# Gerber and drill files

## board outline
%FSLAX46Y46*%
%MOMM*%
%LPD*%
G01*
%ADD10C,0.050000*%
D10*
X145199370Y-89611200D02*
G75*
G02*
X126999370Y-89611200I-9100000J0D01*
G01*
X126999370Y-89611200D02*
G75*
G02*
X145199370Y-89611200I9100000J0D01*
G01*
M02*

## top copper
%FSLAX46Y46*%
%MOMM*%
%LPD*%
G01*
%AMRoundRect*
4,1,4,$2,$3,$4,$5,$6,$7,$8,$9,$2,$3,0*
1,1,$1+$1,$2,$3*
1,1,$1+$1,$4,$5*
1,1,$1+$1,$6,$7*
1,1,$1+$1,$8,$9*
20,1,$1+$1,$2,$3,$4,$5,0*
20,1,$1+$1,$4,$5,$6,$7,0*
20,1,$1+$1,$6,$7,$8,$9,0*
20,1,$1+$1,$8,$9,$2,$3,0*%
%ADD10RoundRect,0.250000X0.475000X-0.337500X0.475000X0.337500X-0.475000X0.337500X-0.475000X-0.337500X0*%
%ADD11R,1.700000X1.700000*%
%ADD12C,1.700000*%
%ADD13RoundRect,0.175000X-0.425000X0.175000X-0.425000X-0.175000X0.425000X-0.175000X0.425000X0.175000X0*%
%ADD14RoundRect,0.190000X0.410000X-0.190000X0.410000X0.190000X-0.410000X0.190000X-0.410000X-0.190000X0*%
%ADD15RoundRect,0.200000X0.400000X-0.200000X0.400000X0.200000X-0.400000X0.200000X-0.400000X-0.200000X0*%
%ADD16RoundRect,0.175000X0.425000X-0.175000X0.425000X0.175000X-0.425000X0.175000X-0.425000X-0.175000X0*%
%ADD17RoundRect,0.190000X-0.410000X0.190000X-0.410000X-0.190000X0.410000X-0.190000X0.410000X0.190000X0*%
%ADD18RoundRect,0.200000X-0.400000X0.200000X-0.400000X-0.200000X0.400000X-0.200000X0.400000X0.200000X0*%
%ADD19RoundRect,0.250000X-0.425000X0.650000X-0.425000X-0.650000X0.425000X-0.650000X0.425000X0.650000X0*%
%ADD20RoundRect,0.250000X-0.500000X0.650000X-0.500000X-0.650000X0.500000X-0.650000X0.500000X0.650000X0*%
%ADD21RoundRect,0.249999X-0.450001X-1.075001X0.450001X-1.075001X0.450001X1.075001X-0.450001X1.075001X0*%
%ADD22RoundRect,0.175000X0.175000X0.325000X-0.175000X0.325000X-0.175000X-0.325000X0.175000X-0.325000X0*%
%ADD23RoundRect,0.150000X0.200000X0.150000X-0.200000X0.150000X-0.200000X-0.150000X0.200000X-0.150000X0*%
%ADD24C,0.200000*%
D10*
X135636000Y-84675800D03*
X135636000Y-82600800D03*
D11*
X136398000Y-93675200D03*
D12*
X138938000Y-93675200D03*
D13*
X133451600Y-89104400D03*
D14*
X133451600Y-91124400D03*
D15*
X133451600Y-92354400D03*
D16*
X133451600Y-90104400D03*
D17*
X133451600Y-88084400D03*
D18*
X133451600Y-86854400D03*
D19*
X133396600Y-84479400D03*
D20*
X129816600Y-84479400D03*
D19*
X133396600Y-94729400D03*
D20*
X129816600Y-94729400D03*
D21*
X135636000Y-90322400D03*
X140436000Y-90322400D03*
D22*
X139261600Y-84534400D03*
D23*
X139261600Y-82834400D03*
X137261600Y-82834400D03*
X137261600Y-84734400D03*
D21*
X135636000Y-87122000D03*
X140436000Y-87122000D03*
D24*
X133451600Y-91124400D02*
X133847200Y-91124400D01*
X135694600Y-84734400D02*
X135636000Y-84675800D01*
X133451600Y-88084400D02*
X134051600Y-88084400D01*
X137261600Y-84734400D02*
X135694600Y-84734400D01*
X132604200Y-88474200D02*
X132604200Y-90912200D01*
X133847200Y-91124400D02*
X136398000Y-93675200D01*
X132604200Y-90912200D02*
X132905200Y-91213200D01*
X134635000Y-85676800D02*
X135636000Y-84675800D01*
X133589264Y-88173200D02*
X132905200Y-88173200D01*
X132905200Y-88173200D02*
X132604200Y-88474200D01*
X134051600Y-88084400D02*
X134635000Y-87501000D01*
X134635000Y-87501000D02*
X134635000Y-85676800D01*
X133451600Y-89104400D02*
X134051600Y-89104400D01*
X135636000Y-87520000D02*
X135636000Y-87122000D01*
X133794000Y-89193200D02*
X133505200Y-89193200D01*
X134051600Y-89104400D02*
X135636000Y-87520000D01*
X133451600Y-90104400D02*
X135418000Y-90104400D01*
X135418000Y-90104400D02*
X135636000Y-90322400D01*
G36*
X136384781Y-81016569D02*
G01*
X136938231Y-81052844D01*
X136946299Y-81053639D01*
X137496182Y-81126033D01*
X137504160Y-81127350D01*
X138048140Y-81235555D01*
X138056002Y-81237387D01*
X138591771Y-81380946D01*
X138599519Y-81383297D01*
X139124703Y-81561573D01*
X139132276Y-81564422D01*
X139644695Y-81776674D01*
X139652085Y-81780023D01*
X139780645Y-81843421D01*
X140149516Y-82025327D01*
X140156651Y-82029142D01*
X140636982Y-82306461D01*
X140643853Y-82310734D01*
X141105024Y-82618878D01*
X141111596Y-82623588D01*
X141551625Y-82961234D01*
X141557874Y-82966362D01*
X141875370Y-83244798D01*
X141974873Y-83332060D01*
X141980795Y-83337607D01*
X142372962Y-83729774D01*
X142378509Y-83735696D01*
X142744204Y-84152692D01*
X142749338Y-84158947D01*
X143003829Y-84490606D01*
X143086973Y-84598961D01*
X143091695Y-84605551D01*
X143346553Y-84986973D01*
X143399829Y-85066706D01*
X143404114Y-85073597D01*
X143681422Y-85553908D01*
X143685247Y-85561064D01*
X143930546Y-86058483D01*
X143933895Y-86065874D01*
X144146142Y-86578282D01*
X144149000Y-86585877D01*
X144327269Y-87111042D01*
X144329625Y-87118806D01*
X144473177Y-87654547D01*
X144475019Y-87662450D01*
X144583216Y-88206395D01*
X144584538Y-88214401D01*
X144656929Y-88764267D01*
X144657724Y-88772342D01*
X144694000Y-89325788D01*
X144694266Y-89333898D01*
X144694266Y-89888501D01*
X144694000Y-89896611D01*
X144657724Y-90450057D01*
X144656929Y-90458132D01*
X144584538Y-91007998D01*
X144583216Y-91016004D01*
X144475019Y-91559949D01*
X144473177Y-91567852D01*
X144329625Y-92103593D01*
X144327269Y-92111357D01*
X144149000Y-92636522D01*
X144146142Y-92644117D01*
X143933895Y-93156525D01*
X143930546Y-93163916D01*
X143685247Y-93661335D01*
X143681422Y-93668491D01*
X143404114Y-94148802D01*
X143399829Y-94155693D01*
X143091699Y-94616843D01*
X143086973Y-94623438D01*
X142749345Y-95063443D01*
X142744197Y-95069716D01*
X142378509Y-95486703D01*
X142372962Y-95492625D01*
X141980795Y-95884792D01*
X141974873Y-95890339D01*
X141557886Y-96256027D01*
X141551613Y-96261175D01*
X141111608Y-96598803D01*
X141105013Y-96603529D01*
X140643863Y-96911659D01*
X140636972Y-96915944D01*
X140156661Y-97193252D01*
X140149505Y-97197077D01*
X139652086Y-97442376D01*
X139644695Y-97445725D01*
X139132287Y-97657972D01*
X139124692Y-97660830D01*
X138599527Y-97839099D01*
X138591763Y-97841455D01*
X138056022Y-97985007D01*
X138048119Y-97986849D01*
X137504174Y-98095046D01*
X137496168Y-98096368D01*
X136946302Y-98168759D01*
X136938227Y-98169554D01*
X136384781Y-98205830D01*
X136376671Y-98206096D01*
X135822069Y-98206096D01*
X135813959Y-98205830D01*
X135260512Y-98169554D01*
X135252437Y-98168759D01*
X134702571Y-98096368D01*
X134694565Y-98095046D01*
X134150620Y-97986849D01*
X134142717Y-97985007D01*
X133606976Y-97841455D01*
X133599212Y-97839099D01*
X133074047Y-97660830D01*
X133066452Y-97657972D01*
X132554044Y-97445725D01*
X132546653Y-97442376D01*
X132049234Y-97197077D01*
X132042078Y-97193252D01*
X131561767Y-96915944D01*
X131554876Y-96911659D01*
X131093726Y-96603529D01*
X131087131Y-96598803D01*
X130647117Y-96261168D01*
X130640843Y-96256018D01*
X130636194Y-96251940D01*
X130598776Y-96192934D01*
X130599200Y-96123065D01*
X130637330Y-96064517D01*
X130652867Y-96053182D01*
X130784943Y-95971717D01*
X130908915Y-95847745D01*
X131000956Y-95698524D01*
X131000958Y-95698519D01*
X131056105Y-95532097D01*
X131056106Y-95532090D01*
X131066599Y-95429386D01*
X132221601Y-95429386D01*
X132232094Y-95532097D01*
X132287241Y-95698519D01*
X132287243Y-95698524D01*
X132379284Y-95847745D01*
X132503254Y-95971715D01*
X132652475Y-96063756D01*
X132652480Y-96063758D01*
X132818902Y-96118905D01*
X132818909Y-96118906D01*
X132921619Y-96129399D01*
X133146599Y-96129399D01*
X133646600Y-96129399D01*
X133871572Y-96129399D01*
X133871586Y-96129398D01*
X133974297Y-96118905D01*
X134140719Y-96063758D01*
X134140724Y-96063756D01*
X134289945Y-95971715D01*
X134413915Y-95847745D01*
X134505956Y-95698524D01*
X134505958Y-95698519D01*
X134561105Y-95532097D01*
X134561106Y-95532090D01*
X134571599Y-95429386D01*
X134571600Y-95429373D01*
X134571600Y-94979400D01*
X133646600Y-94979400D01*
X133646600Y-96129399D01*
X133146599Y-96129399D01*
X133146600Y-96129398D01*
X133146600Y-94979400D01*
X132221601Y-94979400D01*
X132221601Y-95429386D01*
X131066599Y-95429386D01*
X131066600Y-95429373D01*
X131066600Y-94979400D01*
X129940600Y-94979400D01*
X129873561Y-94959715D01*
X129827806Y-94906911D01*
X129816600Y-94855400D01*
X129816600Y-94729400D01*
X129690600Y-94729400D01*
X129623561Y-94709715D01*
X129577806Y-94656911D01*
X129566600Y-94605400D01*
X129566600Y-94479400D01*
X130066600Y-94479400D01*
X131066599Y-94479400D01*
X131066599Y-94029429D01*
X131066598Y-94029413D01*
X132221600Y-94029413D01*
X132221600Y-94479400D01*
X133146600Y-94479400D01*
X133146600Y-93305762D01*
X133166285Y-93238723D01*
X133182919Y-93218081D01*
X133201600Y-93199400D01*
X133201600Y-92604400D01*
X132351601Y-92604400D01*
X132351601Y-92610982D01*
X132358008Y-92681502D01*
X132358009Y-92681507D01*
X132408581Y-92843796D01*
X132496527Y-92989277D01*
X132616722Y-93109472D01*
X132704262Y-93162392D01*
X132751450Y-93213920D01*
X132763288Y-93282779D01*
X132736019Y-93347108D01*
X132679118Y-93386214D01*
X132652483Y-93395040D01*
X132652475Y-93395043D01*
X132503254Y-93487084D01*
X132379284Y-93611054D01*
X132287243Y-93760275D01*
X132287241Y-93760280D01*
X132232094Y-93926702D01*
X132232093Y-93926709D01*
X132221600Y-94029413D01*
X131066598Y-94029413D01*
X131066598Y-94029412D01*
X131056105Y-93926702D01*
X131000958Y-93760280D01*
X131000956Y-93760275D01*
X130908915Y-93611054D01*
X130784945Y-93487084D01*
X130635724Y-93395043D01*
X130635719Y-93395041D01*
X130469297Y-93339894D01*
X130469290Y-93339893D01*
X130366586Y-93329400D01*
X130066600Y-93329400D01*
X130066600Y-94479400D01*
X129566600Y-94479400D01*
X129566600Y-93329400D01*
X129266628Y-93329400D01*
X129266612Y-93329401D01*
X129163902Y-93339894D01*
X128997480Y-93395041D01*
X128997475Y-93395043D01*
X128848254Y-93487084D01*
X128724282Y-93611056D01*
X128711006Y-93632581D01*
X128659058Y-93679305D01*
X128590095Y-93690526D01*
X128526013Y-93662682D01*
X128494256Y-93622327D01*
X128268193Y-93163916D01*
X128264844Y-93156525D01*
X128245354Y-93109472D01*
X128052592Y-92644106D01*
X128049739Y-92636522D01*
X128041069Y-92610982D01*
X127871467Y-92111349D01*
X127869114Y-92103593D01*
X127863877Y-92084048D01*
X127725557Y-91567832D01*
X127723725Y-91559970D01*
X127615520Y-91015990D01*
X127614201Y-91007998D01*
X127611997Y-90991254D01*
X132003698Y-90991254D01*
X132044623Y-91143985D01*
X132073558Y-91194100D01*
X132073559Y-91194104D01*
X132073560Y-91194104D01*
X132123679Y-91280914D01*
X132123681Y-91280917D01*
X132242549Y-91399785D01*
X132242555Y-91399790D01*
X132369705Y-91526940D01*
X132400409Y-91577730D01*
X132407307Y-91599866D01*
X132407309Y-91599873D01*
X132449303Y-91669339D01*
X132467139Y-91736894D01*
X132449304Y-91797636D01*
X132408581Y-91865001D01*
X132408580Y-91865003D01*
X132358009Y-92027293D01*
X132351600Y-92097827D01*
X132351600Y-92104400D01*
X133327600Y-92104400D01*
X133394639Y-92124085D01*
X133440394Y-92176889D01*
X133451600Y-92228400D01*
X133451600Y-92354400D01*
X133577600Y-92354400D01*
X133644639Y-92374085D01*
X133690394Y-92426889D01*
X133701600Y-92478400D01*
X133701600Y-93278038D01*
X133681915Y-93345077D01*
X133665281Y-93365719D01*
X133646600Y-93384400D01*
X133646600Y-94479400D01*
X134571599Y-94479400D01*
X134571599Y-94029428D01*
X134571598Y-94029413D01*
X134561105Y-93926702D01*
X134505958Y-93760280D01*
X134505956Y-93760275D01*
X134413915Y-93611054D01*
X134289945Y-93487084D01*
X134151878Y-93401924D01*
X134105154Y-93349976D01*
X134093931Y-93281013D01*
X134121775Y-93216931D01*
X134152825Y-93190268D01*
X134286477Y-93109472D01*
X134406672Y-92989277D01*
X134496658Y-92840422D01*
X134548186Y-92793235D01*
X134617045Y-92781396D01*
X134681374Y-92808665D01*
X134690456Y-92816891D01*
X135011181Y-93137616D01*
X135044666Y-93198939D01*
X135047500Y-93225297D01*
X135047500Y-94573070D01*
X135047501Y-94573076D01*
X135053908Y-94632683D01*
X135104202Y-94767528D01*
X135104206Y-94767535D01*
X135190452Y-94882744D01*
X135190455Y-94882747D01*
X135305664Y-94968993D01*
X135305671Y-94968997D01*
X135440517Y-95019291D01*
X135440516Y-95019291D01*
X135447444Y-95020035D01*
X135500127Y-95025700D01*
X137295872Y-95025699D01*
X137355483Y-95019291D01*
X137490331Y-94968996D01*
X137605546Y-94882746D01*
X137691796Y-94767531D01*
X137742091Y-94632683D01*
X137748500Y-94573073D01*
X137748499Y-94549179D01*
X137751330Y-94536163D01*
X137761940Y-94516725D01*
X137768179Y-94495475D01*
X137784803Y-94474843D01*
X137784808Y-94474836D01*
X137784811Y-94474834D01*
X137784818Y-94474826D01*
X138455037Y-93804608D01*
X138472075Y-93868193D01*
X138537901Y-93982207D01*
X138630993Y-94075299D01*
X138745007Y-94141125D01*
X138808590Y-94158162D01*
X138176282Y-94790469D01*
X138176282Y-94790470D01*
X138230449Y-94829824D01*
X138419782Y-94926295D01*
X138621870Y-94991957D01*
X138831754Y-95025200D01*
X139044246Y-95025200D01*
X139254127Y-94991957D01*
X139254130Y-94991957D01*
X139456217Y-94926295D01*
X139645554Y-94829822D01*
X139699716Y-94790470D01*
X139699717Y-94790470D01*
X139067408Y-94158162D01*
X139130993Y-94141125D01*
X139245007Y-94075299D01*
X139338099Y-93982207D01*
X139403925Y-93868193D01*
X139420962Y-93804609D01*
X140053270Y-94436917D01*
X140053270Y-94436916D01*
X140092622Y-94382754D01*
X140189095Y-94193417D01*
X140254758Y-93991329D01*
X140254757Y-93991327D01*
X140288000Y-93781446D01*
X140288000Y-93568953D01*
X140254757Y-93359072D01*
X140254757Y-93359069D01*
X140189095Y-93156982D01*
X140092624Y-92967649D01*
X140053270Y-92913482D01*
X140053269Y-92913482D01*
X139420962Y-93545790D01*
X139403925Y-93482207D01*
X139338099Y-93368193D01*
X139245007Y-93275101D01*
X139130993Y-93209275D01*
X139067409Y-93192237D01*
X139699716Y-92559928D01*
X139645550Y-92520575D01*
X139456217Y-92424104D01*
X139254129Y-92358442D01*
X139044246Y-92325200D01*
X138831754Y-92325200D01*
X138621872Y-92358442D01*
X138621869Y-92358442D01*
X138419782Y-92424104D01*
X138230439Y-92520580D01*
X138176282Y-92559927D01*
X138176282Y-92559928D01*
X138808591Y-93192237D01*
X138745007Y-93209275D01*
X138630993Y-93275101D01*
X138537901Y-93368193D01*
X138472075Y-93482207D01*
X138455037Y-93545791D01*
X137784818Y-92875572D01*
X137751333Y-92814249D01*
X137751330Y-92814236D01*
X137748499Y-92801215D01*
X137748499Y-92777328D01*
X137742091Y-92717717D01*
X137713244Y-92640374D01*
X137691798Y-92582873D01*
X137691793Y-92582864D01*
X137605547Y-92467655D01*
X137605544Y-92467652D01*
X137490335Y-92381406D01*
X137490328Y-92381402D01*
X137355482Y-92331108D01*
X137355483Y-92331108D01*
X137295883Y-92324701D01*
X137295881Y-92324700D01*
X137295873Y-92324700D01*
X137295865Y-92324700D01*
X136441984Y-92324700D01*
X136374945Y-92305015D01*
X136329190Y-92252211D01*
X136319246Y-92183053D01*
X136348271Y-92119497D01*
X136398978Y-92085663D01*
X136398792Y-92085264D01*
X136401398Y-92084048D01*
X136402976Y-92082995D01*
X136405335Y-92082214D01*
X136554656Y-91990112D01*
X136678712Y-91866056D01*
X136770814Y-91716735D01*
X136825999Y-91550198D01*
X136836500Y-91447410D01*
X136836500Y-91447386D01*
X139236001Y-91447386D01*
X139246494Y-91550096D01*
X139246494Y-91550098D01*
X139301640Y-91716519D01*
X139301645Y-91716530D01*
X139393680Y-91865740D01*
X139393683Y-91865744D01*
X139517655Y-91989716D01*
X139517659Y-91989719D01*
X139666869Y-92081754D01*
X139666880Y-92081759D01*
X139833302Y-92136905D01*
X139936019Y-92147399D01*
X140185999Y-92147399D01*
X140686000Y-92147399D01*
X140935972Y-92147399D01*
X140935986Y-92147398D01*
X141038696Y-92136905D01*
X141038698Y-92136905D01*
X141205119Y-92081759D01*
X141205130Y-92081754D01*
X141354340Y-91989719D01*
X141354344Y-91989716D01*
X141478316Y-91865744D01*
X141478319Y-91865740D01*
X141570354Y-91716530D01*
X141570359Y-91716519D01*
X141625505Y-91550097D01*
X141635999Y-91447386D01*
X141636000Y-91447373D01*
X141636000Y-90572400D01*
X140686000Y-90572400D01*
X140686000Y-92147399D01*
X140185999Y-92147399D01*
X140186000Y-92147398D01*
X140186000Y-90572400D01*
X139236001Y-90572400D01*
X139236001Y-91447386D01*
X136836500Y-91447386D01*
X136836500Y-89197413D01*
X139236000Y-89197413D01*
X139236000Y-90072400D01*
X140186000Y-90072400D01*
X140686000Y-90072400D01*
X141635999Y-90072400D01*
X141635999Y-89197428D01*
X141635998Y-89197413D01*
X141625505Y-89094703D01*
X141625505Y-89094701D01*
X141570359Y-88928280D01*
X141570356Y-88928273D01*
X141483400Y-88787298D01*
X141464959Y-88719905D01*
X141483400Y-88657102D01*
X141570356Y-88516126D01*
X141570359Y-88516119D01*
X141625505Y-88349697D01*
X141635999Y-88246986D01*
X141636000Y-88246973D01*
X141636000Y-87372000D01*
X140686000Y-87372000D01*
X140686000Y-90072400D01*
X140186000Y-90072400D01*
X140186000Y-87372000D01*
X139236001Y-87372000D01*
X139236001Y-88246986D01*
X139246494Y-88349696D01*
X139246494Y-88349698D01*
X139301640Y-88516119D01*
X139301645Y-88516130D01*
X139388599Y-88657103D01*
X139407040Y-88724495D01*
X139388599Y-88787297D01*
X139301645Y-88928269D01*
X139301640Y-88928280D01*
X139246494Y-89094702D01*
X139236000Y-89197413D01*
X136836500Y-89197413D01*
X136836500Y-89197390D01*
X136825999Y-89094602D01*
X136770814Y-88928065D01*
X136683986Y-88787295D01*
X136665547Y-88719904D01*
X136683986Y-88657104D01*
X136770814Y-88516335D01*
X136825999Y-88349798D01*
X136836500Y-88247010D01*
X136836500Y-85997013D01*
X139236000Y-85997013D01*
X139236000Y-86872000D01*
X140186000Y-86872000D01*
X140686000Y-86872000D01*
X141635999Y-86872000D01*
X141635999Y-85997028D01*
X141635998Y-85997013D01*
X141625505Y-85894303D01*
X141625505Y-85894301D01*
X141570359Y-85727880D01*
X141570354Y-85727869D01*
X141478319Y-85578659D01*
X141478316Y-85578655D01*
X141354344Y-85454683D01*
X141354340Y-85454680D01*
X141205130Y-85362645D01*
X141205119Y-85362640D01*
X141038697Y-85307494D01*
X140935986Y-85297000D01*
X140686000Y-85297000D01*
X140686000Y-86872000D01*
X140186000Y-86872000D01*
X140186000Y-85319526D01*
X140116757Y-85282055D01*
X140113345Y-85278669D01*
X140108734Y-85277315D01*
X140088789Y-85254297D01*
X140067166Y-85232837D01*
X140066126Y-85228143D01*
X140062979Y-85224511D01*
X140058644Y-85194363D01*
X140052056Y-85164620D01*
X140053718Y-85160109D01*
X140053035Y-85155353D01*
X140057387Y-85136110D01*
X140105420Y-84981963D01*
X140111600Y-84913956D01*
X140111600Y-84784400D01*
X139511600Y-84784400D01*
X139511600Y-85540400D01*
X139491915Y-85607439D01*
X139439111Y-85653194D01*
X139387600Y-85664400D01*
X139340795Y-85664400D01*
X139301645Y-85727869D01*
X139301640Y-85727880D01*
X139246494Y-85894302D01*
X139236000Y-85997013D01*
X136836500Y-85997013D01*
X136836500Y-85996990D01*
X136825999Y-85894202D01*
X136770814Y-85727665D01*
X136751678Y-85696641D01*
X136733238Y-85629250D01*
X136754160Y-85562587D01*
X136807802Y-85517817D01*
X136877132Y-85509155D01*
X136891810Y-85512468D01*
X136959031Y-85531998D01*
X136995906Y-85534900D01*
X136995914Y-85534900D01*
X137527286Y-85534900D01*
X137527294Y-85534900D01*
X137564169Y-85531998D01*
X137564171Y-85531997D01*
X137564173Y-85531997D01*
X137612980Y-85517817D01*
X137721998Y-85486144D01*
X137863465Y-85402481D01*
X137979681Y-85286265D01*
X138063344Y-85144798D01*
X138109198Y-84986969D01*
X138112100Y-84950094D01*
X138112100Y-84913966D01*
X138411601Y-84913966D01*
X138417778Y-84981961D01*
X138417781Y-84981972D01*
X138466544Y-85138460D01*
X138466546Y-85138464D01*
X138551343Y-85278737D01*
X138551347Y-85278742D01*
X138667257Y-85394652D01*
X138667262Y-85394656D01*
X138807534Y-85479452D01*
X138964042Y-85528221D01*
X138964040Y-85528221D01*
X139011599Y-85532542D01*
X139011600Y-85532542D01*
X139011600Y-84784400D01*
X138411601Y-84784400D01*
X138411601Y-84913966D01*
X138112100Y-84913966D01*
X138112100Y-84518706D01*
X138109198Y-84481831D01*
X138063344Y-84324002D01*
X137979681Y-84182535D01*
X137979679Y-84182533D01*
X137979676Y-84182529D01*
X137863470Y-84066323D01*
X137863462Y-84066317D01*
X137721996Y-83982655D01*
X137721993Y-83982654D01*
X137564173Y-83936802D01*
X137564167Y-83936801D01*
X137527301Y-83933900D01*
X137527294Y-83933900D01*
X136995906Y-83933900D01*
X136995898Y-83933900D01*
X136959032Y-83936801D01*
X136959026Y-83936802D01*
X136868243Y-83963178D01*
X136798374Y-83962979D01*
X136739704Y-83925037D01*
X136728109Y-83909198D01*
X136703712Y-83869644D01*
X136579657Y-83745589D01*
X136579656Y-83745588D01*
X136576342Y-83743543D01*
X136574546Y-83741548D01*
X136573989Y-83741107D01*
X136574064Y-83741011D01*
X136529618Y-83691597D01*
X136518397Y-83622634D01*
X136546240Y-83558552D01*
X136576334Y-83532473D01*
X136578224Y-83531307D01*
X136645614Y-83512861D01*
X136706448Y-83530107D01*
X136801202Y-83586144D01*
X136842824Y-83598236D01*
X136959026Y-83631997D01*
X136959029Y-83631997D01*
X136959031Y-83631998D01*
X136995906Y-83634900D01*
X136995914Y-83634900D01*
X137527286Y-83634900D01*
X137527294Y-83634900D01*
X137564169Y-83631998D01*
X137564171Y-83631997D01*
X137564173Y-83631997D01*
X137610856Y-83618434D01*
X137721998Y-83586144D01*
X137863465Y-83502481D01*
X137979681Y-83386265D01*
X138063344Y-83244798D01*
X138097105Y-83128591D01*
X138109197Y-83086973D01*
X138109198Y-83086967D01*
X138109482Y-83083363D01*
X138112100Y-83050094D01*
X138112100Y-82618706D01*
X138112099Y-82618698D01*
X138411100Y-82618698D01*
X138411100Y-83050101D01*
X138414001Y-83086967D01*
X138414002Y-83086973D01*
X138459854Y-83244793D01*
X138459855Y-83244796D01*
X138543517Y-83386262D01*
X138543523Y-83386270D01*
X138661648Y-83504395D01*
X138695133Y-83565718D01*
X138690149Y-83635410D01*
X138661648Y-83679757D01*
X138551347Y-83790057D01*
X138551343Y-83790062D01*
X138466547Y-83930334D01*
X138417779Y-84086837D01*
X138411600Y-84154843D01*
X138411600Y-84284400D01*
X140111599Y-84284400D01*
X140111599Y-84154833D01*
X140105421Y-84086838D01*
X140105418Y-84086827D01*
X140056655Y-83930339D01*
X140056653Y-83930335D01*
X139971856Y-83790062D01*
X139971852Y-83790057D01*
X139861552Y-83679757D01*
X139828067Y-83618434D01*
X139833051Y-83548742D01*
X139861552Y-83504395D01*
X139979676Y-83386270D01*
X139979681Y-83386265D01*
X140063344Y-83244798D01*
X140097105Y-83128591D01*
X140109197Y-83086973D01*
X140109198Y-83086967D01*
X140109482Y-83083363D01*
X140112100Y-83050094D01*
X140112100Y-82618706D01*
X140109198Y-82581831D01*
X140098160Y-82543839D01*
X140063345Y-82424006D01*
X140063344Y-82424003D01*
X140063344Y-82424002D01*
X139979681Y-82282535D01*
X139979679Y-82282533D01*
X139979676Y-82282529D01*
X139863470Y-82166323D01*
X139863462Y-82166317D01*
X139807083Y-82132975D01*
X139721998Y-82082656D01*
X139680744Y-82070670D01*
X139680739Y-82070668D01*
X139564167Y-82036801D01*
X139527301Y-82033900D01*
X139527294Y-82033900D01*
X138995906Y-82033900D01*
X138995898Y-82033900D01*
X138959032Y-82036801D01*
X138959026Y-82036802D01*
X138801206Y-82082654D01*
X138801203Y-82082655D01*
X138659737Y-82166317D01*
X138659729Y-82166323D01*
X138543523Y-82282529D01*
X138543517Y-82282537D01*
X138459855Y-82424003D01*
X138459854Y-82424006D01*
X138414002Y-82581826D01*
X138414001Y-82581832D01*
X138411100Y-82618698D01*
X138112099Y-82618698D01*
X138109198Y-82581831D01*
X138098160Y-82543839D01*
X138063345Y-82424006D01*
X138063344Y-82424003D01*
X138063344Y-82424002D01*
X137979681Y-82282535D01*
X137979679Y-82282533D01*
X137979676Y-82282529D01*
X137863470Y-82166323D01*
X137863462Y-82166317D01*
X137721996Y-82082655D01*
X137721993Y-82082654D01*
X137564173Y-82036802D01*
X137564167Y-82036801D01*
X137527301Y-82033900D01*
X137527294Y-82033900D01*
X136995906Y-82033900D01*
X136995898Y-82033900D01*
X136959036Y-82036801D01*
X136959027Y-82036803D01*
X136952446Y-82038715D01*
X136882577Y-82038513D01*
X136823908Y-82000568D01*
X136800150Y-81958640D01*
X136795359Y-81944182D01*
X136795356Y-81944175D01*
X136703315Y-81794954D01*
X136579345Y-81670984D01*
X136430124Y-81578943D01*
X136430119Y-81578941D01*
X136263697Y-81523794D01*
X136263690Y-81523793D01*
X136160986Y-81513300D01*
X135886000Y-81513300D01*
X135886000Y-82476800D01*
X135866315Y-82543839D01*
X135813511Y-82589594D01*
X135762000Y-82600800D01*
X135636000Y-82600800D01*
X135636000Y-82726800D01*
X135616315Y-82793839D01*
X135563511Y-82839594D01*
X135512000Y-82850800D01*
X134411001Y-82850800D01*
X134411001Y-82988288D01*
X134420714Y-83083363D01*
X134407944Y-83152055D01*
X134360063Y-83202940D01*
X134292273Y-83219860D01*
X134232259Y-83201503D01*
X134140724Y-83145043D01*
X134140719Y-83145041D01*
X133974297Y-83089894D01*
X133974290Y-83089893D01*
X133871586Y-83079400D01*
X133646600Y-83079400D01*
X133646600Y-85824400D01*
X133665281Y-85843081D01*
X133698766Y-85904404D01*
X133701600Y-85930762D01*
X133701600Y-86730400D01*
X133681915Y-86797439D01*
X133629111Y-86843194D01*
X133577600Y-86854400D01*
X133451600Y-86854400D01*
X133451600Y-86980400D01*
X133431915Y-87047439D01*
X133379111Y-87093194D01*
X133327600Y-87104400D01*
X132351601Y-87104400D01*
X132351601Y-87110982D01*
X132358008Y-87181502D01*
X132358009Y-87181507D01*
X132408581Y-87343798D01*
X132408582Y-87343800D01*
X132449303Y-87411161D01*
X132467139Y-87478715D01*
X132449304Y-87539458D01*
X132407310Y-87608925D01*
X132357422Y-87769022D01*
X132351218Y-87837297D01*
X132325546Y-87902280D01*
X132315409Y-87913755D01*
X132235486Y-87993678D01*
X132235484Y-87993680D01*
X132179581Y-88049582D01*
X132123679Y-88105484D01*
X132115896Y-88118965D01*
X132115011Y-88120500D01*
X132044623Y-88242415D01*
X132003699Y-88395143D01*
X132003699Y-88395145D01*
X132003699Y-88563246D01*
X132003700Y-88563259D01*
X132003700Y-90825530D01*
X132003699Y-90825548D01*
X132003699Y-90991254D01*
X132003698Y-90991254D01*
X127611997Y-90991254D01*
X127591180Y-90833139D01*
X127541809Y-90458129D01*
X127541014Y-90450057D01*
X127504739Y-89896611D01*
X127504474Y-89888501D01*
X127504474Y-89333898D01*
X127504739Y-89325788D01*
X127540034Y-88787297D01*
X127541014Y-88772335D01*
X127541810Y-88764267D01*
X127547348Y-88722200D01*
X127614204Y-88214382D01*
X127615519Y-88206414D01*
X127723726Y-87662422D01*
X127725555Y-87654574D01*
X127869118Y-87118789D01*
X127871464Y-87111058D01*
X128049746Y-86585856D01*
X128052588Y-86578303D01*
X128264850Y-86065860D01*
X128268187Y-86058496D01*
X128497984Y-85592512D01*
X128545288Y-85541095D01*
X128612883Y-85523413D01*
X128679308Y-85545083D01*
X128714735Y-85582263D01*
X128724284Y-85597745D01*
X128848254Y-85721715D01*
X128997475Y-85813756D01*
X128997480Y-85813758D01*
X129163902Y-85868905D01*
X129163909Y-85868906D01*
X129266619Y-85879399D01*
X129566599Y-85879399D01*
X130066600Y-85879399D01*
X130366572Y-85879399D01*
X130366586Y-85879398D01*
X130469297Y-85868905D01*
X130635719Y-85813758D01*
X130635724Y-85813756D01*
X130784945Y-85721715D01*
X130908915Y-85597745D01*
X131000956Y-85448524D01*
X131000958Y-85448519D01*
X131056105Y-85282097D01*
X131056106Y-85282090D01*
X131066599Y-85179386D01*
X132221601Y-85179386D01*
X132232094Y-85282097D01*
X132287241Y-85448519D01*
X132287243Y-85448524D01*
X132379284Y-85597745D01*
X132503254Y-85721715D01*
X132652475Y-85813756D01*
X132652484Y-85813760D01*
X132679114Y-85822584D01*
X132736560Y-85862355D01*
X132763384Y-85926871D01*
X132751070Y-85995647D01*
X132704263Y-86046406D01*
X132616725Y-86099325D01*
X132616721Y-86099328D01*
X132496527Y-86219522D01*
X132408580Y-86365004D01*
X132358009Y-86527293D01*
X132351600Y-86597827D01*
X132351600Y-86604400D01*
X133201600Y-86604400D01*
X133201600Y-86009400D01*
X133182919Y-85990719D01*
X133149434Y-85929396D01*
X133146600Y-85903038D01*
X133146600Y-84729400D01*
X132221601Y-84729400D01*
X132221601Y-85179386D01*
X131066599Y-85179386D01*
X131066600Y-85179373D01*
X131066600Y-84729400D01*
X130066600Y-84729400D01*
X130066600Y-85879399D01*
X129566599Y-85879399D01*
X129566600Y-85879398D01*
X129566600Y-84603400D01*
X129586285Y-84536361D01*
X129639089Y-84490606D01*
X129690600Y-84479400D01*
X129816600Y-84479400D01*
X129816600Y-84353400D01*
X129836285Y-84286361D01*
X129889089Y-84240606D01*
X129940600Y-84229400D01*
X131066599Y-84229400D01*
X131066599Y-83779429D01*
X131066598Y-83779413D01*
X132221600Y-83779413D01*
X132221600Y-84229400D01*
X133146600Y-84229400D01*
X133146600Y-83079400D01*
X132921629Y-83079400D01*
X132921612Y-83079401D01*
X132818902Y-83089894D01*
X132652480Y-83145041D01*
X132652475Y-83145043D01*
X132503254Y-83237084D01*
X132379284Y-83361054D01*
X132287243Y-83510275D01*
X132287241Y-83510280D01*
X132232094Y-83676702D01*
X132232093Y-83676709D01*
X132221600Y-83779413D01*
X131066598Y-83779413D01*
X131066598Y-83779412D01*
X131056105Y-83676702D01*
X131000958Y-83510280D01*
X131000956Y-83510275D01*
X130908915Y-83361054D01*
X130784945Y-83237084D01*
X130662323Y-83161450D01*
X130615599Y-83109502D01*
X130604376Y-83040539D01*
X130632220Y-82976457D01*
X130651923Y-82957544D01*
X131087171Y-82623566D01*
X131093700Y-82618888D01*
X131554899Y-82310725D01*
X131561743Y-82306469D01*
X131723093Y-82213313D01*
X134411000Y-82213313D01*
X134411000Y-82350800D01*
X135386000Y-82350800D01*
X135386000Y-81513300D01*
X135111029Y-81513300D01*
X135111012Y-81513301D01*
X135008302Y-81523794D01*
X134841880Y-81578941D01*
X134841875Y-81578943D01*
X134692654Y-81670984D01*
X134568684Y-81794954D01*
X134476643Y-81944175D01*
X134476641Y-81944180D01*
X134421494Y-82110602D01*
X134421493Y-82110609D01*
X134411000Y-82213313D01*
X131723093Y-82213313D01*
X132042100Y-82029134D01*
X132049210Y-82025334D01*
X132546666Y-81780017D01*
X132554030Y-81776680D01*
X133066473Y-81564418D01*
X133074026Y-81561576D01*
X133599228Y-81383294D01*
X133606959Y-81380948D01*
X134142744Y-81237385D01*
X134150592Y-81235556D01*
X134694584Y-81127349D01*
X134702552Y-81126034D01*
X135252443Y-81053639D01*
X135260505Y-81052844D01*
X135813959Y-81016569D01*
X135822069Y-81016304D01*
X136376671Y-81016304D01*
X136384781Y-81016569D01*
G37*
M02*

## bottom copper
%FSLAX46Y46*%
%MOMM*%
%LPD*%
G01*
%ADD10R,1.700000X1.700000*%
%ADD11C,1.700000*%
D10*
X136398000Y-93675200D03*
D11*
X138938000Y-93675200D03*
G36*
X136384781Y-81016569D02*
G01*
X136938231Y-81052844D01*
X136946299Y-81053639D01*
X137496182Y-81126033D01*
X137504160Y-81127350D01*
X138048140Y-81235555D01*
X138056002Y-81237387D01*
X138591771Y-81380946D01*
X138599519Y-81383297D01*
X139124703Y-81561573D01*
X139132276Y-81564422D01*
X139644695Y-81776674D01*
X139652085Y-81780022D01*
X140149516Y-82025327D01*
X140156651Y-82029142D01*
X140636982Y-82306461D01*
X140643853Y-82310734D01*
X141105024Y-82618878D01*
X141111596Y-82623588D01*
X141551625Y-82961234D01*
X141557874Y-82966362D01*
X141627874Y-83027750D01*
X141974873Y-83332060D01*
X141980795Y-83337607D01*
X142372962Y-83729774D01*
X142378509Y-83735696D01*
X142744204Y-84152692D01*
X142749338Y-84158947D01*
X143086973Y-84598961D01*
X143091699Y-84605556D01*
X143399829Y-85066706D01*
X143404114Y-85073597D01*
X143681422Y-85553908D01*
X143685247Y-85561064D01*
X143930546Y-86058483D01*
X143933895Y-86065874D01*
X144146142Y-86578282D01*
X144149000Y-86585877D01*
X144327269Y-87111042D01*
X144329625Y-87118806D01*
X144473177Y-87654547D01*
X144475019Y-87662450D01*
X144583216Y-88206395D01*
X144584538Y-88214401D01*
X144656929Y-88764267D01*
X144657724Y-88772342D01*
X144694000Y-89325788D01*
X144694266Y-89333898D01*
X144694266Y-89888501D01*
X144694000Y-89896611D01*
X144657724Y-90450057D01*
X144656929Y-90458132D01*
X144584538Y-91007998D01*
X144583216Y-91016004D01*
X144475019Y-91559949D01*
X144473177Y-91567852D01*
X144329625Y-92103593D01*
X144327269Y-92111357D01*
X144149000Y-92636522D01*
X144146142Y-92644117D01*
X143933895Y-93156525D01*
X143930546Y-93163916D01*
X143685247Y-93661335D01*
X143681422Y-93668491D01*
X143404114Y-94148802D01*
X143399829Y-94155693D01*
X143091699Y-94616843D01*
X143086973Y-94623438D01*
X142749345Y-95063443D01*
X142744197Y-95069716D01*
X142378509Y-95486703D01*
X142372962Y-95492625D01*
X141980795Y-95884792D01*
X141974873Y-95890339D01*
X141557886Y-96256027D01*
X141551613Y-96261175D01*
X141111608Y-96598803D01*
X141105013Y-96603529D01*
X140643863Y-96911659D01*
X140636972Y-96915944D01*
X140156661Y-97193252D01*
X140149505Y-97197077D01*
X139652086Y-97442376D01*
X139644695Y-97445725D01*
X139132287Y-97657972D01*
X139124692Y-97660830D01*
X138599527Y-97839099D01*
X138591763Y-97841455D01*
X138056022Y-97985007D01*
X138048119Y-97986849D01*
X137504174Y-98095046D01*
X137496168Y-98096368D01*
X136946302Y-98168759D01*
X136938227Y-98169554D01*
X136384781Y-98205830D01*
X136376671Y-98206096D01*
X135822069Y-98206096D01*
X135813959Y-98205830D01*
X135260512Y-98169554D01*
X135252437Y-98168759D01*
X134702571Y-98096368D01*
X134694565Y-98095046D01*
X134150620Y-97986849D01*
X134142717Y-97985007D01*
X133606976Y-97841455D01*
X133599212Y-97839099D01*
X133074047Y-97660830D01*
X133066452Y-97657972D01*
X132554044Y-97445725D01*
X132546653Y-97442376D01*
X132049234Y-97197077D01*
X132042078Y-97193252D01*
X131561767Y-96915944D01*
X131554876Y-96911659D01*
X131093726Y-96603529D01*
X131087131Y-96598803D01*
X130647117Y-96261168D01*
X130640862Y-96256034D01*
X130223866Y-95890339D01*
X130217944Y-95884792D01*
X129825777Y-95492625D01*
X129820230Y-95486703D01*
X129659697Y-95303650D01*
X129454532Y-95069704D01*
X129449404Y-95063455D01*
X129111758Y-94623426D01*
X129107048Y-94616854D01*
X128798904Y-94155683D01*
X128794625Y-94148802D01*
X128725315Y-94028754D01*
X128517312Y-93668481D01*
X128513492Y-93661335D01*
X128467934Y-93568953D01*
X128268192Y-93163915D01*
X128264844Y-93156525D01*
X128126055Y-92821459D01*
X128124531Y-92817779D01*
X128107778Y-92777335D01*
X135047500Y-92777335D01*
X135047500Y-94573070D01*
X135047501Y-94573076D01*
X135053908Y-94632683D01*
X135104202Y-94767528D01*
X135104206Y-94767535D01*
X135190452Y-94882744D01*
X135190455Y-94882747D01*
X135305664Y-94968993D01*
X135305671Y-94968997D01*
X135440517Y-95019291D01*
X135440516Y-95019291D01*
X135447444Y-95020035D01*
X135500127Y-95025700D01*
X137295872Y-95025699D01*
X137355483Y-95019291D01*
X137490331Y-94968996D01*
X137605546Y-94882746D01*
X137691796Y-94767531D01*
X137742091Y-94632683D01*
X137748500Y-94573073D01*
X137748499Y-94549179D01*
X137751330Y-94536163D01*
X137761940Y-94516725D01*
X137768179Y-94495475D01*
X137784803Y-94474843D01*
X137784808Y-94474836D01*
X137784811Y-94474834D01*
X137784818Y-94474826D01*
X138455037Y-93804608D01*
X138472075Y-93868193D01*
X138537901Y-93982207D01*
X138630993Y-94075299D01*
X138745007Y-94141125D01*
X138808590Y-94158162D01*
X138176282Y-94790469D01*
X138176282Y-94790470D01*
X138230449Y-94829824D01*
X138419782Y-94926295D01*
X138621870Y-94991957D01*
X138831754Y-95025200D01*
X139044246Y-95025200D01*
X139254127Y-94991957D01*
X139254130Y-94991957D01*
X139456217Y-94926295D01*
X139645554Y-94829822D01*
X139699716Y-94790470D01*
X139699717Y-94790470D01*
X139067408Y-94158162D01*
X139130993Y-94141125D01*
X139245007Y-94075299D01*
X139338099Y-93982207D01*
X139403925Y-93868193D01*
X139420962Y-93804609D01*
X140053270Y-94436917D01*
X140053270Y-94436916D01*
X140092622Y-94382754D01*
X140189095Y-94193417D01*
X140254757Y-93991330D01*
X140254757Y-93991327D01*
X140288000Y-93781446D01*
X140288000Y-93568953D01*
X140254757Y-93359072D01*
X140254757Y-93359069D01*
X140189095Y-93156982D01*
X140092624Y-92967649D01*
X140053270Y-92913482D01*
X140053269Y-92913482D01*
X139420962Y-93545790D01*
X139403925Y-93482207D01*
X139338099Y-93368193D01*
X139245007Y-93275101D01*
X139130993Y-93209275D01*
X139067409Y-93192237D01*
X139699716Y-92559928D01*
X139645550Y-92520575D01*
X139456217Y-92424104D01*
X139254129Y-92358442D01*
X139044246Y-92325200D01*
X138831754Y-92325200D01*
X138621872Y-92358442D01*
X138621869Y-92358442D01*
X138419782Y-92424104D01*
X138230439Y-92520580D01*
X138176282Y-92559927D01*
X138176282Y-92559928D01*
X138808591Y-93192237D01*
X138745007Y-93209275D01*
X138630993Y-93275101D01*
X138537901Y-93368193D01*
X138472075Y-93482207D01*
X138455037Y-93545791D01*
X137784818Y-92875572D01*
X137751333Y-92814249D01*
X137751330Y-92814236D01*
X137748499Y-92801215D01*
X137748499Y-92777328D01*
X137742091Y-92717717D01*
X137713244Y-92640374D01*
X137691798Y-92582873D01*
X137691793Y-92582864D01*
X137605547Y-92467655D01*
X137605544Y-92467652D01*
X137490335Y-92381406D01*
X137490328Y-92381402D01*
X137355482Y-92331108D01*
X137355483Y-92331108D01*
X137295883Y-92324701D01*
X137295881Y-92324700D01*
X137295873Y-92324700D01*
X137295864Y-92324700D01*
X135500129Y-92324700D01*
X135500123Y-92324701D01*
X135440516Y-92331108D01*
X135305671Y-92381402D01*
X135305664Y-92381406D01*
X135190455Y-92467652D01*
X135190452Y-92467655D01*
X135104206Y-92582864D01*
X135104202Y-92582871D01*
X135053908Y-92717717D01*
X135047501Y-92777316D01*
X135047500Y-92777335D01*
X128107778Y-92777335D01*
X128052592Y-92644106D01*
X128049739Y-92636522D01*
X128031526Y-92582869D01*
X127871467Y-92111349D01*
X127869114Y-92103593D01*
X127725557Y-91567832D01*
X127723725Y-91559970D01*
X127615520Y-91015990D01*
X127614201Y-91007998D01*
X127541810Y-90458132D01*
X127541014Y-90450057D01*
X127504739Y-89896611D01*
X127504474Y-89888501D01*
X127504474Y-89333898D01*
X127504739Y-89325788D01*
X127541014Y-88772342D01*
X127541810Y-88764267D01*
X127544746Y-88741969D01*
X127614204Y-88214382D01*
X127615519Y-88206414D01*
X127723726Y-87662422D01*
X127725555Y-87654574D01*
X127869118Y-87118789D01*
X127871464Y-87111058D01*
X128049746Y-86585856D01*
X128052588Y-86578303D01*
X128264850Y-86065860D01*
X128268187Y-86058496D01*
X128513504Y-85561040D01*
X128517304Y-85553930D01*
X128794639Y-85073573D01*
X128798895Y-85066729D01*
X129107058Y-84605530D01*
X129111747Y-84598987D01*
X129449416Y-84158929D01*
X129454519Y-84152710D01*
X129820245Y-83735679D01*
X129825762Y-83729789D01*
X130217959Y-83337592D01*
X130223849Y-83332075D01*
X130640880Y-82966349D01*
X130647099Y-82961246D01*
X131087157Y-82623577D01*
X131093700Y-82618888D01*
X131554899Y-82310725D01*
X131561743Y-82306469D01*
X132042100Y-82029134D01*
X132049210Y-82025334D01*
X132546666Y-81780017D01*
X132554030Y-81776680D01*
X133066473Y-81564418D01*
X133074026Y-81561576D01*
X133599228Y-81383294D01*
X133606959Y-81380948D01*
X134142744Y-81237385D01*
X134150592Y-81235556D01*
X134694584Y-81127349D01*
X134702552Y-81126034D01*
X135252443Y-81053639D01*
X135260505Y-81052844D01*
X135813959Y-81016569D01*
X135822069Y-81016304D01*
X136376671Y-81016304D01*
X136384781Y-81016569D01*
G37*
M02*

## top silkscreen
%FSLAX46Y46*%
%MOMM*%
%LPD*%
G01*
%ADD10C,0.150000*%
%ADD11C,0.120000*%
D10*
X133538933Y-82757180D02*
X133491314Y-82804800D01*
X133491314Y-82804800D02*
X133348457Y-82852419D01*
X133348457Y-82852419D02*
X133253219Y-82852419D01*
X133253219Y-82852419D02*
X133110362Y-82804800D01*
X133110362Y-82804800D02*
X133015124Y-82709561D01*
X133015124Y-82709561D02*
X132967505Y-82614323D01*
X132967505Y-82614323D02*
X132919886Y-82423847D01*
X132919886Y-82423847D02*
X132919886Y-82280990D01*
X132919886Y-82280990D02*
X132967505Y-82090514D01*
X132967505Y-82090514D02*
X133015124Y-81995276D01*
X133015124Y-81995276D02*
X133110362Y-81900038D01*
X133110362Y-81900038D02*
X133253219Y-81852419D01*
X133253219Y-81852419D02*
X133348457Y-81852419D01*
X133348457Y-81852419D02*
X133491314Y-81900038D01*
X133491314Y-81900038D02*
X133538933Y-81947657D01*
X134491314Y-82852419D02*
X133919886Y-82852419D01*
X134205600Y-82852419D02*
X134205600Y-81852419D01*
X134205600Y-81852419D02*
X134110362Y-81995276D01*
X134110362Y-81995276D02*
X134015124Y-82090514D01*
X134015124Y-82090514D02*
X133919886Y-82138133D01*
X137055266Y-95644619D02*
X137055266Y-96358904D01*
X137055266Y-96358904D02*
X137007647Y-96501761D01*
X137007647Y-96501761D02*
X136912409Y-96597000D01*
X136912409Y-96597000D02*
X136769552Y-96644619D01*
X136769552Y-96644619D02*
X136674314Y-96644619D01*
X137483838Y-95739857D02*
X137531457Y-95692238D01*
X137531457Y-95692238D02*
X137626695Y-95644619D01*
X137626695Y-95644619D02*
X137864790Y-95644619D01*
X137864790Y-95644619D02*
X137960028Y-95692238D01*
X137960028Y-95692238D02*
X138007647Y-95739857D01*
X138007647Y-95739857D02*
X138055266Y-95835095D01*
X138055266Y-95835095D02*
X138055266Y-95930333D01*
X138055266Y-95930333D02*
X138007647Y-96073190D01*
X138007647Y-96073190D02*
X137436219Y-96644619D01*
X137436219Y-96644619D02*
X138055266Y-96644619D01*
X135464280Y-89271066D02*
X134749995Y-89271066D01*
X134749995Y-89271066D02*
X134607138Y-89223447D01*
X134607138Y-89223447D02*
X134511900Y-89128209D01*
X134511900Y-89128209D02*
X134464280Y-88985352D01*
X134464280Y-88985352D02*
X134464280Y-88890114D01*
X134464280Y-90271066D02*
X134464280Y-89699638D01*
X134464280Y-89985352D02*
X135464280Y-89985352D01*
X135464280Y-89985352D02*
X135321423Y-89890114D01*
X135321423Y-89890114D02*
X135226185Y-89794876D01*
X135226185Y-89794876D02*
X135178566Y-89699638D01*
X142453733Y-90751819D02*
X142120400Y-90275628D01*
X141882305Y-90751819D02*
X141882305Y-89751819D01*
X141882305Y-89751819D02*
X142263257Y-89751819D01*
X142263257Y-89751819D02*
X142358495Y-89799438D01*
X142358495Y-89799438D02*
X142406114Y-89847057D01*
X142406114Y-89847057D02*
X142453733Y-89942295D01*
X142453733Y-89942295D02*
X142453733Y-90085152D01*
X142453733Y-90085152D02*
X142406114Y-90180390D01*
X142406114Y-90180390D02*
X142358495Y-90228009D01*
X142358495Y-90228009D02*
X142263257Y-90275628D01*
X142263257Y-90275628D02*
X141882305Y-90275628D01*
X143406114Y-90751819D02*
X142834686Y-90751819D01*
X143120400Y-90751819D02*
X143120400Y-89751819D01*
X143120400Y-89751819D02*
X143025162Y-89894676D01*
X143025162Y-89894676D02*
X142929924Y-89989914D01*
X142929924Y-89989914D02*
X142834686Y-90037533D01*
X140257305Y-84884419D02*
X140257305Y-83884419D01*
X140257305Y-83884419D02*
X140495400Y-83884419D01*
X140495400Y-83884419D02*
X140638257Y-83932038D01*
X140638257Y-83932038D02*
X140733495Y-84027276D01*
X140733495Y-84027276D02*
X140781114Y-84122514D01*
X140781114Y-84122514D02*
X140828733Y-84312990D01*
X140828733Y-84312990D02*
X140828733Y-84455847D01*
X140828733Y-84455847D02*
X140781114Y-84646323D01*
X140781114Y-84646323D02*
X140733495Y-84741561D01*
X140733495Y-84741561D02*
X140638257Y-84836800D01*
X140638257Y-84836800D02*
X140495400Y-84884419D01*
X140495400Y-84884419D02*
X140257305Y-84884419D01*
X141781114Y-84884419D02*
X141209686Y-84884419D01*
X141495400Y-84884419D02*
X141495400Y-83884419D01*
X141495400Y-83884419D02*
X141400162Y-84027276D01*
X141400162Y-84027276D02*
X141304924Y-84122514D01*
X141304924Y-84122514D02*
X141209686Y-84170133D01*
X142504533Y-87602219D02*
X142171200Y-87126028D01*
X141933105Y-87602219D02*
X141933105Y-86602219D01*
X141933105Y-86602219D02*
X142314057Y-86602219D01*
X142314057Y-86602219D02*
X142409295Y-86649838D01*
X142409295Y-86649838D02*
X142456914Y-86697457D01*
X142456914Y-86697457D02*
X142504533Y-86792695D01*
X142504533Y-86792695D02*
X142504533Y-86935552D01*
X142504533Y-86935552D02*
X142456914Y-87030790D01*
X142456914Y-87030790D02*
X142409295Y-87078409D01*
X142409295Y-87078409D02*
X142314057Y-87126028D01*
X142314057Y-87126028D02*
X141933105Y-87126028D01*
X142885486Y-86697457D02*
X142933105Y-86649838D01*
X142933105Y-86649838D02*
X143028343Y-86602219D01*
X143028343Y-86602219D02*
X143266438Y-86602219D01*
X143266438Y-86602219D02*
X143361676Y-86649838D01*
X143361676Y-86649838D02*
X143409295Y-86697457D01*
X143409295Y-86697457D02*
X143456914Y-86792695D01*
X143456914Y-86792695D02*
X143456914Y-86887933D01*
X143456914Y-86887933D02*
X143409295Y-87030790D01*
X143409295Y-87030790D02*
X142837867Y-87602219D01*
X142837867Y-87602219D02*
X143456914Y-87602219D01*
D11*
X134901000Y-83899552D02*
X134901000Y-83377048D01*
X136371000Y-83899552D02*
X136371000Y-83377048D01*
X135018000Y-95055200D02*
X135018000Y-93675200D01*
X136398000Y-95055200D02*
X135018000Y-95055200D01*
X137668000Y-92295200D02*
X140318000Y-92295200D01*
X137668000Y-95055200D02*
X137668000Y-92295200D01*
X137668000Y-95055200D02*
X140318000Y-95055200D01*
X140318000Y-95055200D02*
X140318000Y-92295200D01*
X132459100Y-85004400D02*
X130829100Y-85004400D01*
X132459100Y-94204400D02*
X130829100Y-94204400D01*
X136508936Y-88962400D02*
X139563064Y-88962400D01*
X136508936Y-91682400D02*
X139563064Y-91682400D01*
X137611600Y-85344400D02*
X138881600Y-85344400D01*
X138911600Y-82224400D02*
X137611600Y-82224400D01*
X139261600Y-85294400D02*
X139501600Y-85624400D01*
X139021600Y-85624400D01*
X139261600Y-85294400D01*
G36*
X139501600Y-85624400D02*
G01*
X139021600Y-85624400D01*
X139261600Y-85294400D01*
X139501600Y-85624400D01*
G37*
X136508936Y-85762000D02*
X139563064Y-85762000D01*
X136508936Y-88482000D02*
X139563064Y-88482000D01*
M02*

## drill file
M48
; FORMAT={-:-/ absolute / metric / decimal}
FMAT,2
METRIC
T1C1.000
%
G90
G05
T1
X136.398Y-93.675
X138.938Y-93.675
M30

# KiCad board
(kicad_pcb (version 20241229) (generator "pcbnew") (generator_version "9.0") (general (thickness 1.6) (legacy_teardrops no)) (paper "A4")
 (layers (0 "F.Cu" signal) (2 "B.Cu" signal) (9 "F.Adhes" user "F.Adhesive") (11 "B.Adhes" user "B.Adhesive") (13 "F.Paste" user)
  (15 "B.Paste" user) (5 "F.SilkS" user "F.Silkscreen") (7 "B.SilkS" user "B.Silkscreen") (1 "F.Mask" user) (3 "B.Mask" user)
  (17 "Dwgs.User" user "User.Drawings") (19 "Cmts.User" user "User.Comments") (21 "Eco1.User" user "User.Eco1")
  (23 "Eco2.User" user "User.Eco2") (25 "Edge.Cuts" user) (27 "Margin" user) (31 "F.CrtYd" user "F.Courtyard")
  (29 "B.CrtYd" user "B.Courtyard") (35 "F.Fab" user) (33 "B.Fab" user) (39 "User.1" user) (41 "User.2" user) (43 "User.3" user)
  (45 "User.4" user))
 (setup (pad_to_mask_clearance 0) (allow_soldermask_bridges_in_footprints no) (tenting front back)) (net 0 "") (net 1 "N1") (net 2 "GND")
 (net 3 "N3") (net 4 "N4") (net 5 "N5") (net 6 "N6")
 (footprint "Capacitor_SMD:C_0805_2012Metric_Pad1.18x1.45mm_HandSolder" (layer "F.Cu") (at 135.636 83.6383 90)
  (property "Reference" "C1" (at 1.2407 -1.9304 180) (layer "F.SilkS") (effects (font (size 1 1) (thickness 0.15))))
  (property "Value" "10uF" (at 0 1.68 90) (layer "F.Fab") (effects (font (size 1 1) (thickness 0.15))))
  (fp_line (start -0.261252 -0.735) (end 0.261252 -0.735) (stroke (width 0.12) (type solid)) (layer "F.SilkS"))
  (fp_line (start -0.261252 0.735) (end 0.261252 0.735) (stroke (width 0.12) (type solid)) (layer "F.SilkS"))
  (pad "1" smd roundrect (at -1.0375 0 90) (size 1.175 1.45) (layers "F.Cu" "F.Mask" "F.Paste") (roundrect_rratio 0.212766) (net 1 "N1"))
  (pad "2" smd roundrect (at 1.0375 0 90) (size 1.175 1.45) (layers "F.Cu" "F.Mask" "F.Paste") (roundrect_rratio 0.212766) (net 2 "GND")))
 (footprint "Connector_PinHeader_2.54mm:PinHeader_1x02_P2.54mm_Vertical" (layer "F.Cu") (at 136.398 93.6752 90)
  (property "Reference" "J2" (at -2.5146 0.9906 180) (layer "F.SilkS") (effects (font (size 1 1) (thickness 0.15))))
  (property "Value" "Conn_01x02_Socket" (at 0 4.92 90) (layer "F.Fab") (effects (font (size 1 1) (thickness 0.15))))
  (fp_line (start -1.38 -1.38) (end 0 -1.38) (stroke (width 0.12) (type solid)) (layer "F.SilkS"))
  (fp_line (start -1.38 0) (end -1.38 -1.38) (stroke (width 0.12) (type solid)) (layer "F.SilkS"))
  (fp_line (start 1.38 1.27) (end 1.38 3.92) (stroke (width 0.12) (type solid)) (layer "F.SilkS"))
  (fp_line (start -1.38 1.27) (end 1.38 1.27) (stroke (width 0.12) (type solid)) (layer "F.SilkS"))
  (fp_line (start -1.38 1.27) (end -1.38 3.92) (stroke (width 0.12) (type solid)) (layer "F.SilkS"))
  (fp_line (start -1.38 3.92) (end 1.38 3.92) (stroke (width 0.12) (type solid)) (layer "F.SilkS"))
  (pad "1" thru_hole rect (at 0 0 90) (size 1.7 1.7) (drill 1) (layers "*.Cu" "*.Mask") (remove_unused_layers no) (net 1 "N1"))
  (pad "2" thru_hole circle (at 0 2.54 90) (size 1.7 1.7) (drill 1) (layers "*.Cu" "*.Mask") (remove_unused_layers no) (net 2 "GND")))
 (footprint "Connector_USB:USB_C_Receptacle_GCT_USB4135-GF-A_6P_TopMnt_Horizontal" (layer "F.Cu") (at 130.4191 89.6044 -90)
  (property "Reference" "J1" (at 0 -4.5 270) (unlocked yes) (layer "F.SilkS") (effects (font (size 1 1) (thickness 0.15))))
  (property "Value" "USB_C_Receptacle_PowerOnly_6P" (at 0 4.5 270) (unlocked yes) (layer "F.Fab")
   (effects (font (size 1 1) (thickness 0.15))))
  (fp_line (start -4.6 -2.04) (end -4.6 -0.41) (stroke (width 0.12) (type solid)) (layer "F.SilkS"))
  (fp_line (start 4.6 -2.04) (end 4.6 -0.41) (stroke (width 0.12) (type solid)) (layer "F.SilkS"))
  (pad "A5" smd roundrect (at -0.5 -3.0325 270) (size 0.7 1.2) (layers "F.Cu" "F.Mask" "F.Paste") (roundrect_rratio 0.25) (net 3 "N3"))
  (pad "A9" smd roundrect (at 1.52 -3.0325 90) (size 0.76 1.2) (layers "F.Cu" "F.Mask" "F.Paste") (roundrect_rratio 0.25) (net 1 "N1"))
  (pad "A12" smd roundrect (at 2.75 -3.0325 90) (size 0.8 1.2) (layers "F.Cu" "F.Mask" "F.Paste") (roundrect_rratio 0.25) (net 2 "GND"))
  (pad "B5" smd roundrect (at 0.5 -3.0325 90) (size 0.7 1.2) (layers "F.Cu" "F.Mask" "F.Paste") (roundrect_rratio 0.25) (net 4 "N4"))
  (pad "B9" smd roundrect (at -1.52 -3.0325 270) (size 0.76 1.2) (layers "F.Cu" "F.Mask" "F.Paste") (roundrect_rratio 0.25) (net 1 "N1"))
  (pad "B12" smd roundrect (at -2.75 -3.0325 270) (size 0.8 1.2) (layers "F.Cu" "F.Mask" "F.Paste") (roundrect_rratio 0.25) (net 2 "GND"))
  (pad "S1" smd roundrect (at -5.125 -2.9775 270) (size 1.8 1.35) (layers "F.Cu" "F.Mask" "F.Paste") (roundrect_rratio 0.1851851852)
   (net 2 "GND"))
  (pad "S1" smd roundrect (at -5.125 0.6025 270) (size 1.8 1.5) (layers "F.Cu" "F.Mask" "F.Paste") (roundrect_rratio 0.1666666667)
   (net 2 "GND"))
  (pad "S1" smd roundrect (at 5.125 -2.9775 270) (size 1.8 1.35) (layers "F.Cu" "F.Mask" "F.Paste") (roundrect_rratio 0.1851851852)
   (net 2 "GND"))
  (pad "S1" smd roundrect (at 5.125 0.6025 270) (size 1.8 1.5) (layers "F.Cu" "F.Mask" "F.Paste") (roundrect_rratio 0.1666666667)
   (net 2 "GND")))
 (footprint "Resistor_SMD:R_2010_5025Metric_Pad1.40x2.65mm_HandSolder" (layer "F.Cu") (at 138.036 90.3224)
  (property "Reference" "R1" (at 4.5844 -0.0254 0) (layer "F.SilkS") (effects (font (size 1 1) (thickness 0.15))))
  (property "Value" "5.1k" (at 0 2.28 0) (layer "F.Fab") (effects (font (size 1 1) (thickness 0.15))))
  (fp_line (start -1.527064 -1.36) (end 1.527064 -1.36) (stroke (width 0.12) (type solid)) (layer "F.SilkS"))
  (fp_line (start -1.527064 1.36) (end 1.527064 1.36) (stroke (width 0.12) (type solid)) (layer "F.SilkS"))
  (pad "1" smd roundrect (at -2.4 0) (size 1.4 2.65) (layers "F.Cu" "F.Mask" "F.Paste") (roundrect_rratio 0.178571) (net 4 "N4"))
  (pad "2" smd roundrect (at 2.4 0) (size 1.4 2.65) (layers "F.Cu" "F.Mask" "F.Paste") (roundrect_rratio 0.178571) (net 2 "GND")))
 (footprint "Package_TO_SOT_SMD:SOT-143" (layer "F.Cu") (at 138.2616 83.7844 180)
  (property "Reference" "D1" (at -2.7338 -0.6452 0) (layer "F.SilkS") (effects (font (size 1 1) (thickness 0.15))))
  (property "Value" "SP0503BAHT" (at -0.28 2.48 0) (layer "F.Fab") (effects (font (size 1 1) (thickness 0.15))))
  (fp_line (start 0.65 -1.56) (end -0.62 -1.56) (stroke (width 0.12) (type solid)) (layer "F.SilkS"))
  (fp_line (start -0.65 1.56) (end 0.65 1.56) (stroke (width 0.12) (type solid)) (layer "F.SilkS"))
  (fp_poly
   (pts (xy -1 -1.51) (xy -1.24 -1.84) (xy -0.76 -1.84) (xy -1 -1.51)) (stroke (width 0.12) (type solid)) (fill yes) (layer "F.SilkS"))
  (pad "1" smd roundrect (at -1 -0.75 180) (size 0.7 1) (layers "F.Cu" "F.Mask" "F.Paste") (roundrect_rratio 0.25) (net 2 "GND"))
  (pad "2" smd roundrect (at -1 0.95 180) (size 0.7 0.6) (layers "F.Cu" "F.Mask" "F.Paste") (roundrect_rratio 0.25) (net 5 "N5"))
  (pad "3" smd roundrect (at 1 0.95 180) (size 0.7 0.6) (layers "F.Cu" "F.Mask" "F.Paste") (roundrect_rratio 0.25) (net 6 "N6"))
  (pad "4" smd roundrect (at 1 -0.95 180) (size 0.7 0.6) (layers "F.Cu" "F.Mask" "F.Paste") (roundrect_rratio 0.25) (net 1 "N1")))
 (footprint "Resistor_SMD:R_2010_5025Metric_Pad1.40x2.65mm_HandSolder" (layer "F.Cu") (at 138.036 87.122)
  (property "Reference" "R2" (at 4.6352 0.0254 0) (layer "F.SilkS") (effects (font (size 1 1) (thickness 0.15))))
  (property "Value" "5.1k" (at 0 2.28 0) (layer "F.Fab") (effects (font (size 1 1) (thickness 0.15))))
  (fp_line (start -1.527064 -1.36) (end 1.527064 -1.36) (stroke (width 0.12) (type solid)) (layer "F.SilkS"))
  (fp_line (start -1.527064 1.36) (end 1.527064 1.36) (stroke (width 0.12) (type solid)) (layer "F.SilkS"))
  (pad "1" smd roundrect (at -2.4 0) (size 1.4 2.65) (layers "F.Cu" "F.Mask" "F.Paste") (roundrect_rratio 0.178571) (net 3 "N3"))
  (pad "2" smd roundrect (at 2.4 0) (size 1.4 2.65) (layers "F.Cu" "F.Mask" "F.Paste") (roundrect_rratio 0.178571) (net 2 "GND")))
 (gr_circle (center 136.09937 89.6112) (end 145.19937 89.6112) (stroke (width 0.05) (type solid)) (fill no) (layer "Edge.Cuts"))
 (segment (start 133.4516 91.1244) (end 133.8472 91.1244) (width 0.2) (layer "F.Cu") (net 1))
 (segment (start 135.6946 84.7344) (end 135.636 84.6758) (width 0.2) (layer "F.Cu") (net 1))
 (segment (start 133.4516 88.0844) (end 134.0516 88.0844) (width 0.2) (layer "F.Cu") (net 1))
 (segment (start 137.2616 84.7344) (end 135.6946 84.7344) (width 0.2) (layer "F.Cu") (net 1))
 (segment (start 132.6042 88.4742) (end 132.6042 90.9122) (width 0.2) (layer "F.Cu") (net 1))
 (segment (start 133.8472 91.1244) (end 136.398 93.6752) (width 0.2) (layer "F.Cu") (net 1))
 (segment (start 132.6042 90.9122) (end 132.9052 91.2132) (width 0.2) (layer "F.Cu") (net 1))
 (segment (start 134.635 85.6768) (end 135.636 84.6758) (width 0.2) (layer "F.Cu") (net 1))
 (segment (start 133.589264 88.1732) (end 132.9052 88.1732) (width 0.2) (layer "F.Cu") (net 1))
 (segment (start 132.9052 88.1732) (end 132.6042 88.4742) (width 0.2) (layer "F.Cu") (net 1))
 (segment (start 134.0516 88.0844) (end 134.635 87.501) (width 0.2) (layer "F.Cu") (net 1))
 (segment (start 134.635 87.501) (end 134.635 85.6768) (width 0.2) (layer "F.Cu") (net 1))
 (segment (start 133.4516 89.1044) (end 134.0516 89.1044) (width 0.2) (layer "F.Cu") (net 3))
 (segment (start 135.636 87.52) (end 135.636 87.122) (width 0.2) (layer "F.Cu") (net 3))
 (segment (start 133.794 89.1932) (end 133.5052 89.1932) (width 0.2) (layer "F.Cu") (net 3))
 (segment (start 134.0516 89.1044) (end 135.636 87.52) (width 0.2) (layer "F.Cu") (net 3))
 (segment (start 133.4516 90.1044) (end 135.418 90.1044) (width 0.2) (layer "F.Cu") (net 4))
 (segment (start 135.418 90.1044) (end 135.636 90.3224) (width 0.2) (layer "F.Cu") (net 4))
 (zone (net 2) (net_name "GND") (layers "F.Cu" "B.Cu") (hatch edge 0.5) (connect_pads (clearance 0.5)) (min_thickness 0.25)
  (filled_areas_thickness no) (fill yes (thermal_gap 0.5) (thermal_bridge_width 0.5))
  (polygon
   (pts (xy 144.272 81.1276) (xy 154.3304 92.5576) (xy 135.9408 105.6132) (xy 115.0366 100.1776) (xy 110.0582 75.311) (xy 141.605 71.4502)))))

